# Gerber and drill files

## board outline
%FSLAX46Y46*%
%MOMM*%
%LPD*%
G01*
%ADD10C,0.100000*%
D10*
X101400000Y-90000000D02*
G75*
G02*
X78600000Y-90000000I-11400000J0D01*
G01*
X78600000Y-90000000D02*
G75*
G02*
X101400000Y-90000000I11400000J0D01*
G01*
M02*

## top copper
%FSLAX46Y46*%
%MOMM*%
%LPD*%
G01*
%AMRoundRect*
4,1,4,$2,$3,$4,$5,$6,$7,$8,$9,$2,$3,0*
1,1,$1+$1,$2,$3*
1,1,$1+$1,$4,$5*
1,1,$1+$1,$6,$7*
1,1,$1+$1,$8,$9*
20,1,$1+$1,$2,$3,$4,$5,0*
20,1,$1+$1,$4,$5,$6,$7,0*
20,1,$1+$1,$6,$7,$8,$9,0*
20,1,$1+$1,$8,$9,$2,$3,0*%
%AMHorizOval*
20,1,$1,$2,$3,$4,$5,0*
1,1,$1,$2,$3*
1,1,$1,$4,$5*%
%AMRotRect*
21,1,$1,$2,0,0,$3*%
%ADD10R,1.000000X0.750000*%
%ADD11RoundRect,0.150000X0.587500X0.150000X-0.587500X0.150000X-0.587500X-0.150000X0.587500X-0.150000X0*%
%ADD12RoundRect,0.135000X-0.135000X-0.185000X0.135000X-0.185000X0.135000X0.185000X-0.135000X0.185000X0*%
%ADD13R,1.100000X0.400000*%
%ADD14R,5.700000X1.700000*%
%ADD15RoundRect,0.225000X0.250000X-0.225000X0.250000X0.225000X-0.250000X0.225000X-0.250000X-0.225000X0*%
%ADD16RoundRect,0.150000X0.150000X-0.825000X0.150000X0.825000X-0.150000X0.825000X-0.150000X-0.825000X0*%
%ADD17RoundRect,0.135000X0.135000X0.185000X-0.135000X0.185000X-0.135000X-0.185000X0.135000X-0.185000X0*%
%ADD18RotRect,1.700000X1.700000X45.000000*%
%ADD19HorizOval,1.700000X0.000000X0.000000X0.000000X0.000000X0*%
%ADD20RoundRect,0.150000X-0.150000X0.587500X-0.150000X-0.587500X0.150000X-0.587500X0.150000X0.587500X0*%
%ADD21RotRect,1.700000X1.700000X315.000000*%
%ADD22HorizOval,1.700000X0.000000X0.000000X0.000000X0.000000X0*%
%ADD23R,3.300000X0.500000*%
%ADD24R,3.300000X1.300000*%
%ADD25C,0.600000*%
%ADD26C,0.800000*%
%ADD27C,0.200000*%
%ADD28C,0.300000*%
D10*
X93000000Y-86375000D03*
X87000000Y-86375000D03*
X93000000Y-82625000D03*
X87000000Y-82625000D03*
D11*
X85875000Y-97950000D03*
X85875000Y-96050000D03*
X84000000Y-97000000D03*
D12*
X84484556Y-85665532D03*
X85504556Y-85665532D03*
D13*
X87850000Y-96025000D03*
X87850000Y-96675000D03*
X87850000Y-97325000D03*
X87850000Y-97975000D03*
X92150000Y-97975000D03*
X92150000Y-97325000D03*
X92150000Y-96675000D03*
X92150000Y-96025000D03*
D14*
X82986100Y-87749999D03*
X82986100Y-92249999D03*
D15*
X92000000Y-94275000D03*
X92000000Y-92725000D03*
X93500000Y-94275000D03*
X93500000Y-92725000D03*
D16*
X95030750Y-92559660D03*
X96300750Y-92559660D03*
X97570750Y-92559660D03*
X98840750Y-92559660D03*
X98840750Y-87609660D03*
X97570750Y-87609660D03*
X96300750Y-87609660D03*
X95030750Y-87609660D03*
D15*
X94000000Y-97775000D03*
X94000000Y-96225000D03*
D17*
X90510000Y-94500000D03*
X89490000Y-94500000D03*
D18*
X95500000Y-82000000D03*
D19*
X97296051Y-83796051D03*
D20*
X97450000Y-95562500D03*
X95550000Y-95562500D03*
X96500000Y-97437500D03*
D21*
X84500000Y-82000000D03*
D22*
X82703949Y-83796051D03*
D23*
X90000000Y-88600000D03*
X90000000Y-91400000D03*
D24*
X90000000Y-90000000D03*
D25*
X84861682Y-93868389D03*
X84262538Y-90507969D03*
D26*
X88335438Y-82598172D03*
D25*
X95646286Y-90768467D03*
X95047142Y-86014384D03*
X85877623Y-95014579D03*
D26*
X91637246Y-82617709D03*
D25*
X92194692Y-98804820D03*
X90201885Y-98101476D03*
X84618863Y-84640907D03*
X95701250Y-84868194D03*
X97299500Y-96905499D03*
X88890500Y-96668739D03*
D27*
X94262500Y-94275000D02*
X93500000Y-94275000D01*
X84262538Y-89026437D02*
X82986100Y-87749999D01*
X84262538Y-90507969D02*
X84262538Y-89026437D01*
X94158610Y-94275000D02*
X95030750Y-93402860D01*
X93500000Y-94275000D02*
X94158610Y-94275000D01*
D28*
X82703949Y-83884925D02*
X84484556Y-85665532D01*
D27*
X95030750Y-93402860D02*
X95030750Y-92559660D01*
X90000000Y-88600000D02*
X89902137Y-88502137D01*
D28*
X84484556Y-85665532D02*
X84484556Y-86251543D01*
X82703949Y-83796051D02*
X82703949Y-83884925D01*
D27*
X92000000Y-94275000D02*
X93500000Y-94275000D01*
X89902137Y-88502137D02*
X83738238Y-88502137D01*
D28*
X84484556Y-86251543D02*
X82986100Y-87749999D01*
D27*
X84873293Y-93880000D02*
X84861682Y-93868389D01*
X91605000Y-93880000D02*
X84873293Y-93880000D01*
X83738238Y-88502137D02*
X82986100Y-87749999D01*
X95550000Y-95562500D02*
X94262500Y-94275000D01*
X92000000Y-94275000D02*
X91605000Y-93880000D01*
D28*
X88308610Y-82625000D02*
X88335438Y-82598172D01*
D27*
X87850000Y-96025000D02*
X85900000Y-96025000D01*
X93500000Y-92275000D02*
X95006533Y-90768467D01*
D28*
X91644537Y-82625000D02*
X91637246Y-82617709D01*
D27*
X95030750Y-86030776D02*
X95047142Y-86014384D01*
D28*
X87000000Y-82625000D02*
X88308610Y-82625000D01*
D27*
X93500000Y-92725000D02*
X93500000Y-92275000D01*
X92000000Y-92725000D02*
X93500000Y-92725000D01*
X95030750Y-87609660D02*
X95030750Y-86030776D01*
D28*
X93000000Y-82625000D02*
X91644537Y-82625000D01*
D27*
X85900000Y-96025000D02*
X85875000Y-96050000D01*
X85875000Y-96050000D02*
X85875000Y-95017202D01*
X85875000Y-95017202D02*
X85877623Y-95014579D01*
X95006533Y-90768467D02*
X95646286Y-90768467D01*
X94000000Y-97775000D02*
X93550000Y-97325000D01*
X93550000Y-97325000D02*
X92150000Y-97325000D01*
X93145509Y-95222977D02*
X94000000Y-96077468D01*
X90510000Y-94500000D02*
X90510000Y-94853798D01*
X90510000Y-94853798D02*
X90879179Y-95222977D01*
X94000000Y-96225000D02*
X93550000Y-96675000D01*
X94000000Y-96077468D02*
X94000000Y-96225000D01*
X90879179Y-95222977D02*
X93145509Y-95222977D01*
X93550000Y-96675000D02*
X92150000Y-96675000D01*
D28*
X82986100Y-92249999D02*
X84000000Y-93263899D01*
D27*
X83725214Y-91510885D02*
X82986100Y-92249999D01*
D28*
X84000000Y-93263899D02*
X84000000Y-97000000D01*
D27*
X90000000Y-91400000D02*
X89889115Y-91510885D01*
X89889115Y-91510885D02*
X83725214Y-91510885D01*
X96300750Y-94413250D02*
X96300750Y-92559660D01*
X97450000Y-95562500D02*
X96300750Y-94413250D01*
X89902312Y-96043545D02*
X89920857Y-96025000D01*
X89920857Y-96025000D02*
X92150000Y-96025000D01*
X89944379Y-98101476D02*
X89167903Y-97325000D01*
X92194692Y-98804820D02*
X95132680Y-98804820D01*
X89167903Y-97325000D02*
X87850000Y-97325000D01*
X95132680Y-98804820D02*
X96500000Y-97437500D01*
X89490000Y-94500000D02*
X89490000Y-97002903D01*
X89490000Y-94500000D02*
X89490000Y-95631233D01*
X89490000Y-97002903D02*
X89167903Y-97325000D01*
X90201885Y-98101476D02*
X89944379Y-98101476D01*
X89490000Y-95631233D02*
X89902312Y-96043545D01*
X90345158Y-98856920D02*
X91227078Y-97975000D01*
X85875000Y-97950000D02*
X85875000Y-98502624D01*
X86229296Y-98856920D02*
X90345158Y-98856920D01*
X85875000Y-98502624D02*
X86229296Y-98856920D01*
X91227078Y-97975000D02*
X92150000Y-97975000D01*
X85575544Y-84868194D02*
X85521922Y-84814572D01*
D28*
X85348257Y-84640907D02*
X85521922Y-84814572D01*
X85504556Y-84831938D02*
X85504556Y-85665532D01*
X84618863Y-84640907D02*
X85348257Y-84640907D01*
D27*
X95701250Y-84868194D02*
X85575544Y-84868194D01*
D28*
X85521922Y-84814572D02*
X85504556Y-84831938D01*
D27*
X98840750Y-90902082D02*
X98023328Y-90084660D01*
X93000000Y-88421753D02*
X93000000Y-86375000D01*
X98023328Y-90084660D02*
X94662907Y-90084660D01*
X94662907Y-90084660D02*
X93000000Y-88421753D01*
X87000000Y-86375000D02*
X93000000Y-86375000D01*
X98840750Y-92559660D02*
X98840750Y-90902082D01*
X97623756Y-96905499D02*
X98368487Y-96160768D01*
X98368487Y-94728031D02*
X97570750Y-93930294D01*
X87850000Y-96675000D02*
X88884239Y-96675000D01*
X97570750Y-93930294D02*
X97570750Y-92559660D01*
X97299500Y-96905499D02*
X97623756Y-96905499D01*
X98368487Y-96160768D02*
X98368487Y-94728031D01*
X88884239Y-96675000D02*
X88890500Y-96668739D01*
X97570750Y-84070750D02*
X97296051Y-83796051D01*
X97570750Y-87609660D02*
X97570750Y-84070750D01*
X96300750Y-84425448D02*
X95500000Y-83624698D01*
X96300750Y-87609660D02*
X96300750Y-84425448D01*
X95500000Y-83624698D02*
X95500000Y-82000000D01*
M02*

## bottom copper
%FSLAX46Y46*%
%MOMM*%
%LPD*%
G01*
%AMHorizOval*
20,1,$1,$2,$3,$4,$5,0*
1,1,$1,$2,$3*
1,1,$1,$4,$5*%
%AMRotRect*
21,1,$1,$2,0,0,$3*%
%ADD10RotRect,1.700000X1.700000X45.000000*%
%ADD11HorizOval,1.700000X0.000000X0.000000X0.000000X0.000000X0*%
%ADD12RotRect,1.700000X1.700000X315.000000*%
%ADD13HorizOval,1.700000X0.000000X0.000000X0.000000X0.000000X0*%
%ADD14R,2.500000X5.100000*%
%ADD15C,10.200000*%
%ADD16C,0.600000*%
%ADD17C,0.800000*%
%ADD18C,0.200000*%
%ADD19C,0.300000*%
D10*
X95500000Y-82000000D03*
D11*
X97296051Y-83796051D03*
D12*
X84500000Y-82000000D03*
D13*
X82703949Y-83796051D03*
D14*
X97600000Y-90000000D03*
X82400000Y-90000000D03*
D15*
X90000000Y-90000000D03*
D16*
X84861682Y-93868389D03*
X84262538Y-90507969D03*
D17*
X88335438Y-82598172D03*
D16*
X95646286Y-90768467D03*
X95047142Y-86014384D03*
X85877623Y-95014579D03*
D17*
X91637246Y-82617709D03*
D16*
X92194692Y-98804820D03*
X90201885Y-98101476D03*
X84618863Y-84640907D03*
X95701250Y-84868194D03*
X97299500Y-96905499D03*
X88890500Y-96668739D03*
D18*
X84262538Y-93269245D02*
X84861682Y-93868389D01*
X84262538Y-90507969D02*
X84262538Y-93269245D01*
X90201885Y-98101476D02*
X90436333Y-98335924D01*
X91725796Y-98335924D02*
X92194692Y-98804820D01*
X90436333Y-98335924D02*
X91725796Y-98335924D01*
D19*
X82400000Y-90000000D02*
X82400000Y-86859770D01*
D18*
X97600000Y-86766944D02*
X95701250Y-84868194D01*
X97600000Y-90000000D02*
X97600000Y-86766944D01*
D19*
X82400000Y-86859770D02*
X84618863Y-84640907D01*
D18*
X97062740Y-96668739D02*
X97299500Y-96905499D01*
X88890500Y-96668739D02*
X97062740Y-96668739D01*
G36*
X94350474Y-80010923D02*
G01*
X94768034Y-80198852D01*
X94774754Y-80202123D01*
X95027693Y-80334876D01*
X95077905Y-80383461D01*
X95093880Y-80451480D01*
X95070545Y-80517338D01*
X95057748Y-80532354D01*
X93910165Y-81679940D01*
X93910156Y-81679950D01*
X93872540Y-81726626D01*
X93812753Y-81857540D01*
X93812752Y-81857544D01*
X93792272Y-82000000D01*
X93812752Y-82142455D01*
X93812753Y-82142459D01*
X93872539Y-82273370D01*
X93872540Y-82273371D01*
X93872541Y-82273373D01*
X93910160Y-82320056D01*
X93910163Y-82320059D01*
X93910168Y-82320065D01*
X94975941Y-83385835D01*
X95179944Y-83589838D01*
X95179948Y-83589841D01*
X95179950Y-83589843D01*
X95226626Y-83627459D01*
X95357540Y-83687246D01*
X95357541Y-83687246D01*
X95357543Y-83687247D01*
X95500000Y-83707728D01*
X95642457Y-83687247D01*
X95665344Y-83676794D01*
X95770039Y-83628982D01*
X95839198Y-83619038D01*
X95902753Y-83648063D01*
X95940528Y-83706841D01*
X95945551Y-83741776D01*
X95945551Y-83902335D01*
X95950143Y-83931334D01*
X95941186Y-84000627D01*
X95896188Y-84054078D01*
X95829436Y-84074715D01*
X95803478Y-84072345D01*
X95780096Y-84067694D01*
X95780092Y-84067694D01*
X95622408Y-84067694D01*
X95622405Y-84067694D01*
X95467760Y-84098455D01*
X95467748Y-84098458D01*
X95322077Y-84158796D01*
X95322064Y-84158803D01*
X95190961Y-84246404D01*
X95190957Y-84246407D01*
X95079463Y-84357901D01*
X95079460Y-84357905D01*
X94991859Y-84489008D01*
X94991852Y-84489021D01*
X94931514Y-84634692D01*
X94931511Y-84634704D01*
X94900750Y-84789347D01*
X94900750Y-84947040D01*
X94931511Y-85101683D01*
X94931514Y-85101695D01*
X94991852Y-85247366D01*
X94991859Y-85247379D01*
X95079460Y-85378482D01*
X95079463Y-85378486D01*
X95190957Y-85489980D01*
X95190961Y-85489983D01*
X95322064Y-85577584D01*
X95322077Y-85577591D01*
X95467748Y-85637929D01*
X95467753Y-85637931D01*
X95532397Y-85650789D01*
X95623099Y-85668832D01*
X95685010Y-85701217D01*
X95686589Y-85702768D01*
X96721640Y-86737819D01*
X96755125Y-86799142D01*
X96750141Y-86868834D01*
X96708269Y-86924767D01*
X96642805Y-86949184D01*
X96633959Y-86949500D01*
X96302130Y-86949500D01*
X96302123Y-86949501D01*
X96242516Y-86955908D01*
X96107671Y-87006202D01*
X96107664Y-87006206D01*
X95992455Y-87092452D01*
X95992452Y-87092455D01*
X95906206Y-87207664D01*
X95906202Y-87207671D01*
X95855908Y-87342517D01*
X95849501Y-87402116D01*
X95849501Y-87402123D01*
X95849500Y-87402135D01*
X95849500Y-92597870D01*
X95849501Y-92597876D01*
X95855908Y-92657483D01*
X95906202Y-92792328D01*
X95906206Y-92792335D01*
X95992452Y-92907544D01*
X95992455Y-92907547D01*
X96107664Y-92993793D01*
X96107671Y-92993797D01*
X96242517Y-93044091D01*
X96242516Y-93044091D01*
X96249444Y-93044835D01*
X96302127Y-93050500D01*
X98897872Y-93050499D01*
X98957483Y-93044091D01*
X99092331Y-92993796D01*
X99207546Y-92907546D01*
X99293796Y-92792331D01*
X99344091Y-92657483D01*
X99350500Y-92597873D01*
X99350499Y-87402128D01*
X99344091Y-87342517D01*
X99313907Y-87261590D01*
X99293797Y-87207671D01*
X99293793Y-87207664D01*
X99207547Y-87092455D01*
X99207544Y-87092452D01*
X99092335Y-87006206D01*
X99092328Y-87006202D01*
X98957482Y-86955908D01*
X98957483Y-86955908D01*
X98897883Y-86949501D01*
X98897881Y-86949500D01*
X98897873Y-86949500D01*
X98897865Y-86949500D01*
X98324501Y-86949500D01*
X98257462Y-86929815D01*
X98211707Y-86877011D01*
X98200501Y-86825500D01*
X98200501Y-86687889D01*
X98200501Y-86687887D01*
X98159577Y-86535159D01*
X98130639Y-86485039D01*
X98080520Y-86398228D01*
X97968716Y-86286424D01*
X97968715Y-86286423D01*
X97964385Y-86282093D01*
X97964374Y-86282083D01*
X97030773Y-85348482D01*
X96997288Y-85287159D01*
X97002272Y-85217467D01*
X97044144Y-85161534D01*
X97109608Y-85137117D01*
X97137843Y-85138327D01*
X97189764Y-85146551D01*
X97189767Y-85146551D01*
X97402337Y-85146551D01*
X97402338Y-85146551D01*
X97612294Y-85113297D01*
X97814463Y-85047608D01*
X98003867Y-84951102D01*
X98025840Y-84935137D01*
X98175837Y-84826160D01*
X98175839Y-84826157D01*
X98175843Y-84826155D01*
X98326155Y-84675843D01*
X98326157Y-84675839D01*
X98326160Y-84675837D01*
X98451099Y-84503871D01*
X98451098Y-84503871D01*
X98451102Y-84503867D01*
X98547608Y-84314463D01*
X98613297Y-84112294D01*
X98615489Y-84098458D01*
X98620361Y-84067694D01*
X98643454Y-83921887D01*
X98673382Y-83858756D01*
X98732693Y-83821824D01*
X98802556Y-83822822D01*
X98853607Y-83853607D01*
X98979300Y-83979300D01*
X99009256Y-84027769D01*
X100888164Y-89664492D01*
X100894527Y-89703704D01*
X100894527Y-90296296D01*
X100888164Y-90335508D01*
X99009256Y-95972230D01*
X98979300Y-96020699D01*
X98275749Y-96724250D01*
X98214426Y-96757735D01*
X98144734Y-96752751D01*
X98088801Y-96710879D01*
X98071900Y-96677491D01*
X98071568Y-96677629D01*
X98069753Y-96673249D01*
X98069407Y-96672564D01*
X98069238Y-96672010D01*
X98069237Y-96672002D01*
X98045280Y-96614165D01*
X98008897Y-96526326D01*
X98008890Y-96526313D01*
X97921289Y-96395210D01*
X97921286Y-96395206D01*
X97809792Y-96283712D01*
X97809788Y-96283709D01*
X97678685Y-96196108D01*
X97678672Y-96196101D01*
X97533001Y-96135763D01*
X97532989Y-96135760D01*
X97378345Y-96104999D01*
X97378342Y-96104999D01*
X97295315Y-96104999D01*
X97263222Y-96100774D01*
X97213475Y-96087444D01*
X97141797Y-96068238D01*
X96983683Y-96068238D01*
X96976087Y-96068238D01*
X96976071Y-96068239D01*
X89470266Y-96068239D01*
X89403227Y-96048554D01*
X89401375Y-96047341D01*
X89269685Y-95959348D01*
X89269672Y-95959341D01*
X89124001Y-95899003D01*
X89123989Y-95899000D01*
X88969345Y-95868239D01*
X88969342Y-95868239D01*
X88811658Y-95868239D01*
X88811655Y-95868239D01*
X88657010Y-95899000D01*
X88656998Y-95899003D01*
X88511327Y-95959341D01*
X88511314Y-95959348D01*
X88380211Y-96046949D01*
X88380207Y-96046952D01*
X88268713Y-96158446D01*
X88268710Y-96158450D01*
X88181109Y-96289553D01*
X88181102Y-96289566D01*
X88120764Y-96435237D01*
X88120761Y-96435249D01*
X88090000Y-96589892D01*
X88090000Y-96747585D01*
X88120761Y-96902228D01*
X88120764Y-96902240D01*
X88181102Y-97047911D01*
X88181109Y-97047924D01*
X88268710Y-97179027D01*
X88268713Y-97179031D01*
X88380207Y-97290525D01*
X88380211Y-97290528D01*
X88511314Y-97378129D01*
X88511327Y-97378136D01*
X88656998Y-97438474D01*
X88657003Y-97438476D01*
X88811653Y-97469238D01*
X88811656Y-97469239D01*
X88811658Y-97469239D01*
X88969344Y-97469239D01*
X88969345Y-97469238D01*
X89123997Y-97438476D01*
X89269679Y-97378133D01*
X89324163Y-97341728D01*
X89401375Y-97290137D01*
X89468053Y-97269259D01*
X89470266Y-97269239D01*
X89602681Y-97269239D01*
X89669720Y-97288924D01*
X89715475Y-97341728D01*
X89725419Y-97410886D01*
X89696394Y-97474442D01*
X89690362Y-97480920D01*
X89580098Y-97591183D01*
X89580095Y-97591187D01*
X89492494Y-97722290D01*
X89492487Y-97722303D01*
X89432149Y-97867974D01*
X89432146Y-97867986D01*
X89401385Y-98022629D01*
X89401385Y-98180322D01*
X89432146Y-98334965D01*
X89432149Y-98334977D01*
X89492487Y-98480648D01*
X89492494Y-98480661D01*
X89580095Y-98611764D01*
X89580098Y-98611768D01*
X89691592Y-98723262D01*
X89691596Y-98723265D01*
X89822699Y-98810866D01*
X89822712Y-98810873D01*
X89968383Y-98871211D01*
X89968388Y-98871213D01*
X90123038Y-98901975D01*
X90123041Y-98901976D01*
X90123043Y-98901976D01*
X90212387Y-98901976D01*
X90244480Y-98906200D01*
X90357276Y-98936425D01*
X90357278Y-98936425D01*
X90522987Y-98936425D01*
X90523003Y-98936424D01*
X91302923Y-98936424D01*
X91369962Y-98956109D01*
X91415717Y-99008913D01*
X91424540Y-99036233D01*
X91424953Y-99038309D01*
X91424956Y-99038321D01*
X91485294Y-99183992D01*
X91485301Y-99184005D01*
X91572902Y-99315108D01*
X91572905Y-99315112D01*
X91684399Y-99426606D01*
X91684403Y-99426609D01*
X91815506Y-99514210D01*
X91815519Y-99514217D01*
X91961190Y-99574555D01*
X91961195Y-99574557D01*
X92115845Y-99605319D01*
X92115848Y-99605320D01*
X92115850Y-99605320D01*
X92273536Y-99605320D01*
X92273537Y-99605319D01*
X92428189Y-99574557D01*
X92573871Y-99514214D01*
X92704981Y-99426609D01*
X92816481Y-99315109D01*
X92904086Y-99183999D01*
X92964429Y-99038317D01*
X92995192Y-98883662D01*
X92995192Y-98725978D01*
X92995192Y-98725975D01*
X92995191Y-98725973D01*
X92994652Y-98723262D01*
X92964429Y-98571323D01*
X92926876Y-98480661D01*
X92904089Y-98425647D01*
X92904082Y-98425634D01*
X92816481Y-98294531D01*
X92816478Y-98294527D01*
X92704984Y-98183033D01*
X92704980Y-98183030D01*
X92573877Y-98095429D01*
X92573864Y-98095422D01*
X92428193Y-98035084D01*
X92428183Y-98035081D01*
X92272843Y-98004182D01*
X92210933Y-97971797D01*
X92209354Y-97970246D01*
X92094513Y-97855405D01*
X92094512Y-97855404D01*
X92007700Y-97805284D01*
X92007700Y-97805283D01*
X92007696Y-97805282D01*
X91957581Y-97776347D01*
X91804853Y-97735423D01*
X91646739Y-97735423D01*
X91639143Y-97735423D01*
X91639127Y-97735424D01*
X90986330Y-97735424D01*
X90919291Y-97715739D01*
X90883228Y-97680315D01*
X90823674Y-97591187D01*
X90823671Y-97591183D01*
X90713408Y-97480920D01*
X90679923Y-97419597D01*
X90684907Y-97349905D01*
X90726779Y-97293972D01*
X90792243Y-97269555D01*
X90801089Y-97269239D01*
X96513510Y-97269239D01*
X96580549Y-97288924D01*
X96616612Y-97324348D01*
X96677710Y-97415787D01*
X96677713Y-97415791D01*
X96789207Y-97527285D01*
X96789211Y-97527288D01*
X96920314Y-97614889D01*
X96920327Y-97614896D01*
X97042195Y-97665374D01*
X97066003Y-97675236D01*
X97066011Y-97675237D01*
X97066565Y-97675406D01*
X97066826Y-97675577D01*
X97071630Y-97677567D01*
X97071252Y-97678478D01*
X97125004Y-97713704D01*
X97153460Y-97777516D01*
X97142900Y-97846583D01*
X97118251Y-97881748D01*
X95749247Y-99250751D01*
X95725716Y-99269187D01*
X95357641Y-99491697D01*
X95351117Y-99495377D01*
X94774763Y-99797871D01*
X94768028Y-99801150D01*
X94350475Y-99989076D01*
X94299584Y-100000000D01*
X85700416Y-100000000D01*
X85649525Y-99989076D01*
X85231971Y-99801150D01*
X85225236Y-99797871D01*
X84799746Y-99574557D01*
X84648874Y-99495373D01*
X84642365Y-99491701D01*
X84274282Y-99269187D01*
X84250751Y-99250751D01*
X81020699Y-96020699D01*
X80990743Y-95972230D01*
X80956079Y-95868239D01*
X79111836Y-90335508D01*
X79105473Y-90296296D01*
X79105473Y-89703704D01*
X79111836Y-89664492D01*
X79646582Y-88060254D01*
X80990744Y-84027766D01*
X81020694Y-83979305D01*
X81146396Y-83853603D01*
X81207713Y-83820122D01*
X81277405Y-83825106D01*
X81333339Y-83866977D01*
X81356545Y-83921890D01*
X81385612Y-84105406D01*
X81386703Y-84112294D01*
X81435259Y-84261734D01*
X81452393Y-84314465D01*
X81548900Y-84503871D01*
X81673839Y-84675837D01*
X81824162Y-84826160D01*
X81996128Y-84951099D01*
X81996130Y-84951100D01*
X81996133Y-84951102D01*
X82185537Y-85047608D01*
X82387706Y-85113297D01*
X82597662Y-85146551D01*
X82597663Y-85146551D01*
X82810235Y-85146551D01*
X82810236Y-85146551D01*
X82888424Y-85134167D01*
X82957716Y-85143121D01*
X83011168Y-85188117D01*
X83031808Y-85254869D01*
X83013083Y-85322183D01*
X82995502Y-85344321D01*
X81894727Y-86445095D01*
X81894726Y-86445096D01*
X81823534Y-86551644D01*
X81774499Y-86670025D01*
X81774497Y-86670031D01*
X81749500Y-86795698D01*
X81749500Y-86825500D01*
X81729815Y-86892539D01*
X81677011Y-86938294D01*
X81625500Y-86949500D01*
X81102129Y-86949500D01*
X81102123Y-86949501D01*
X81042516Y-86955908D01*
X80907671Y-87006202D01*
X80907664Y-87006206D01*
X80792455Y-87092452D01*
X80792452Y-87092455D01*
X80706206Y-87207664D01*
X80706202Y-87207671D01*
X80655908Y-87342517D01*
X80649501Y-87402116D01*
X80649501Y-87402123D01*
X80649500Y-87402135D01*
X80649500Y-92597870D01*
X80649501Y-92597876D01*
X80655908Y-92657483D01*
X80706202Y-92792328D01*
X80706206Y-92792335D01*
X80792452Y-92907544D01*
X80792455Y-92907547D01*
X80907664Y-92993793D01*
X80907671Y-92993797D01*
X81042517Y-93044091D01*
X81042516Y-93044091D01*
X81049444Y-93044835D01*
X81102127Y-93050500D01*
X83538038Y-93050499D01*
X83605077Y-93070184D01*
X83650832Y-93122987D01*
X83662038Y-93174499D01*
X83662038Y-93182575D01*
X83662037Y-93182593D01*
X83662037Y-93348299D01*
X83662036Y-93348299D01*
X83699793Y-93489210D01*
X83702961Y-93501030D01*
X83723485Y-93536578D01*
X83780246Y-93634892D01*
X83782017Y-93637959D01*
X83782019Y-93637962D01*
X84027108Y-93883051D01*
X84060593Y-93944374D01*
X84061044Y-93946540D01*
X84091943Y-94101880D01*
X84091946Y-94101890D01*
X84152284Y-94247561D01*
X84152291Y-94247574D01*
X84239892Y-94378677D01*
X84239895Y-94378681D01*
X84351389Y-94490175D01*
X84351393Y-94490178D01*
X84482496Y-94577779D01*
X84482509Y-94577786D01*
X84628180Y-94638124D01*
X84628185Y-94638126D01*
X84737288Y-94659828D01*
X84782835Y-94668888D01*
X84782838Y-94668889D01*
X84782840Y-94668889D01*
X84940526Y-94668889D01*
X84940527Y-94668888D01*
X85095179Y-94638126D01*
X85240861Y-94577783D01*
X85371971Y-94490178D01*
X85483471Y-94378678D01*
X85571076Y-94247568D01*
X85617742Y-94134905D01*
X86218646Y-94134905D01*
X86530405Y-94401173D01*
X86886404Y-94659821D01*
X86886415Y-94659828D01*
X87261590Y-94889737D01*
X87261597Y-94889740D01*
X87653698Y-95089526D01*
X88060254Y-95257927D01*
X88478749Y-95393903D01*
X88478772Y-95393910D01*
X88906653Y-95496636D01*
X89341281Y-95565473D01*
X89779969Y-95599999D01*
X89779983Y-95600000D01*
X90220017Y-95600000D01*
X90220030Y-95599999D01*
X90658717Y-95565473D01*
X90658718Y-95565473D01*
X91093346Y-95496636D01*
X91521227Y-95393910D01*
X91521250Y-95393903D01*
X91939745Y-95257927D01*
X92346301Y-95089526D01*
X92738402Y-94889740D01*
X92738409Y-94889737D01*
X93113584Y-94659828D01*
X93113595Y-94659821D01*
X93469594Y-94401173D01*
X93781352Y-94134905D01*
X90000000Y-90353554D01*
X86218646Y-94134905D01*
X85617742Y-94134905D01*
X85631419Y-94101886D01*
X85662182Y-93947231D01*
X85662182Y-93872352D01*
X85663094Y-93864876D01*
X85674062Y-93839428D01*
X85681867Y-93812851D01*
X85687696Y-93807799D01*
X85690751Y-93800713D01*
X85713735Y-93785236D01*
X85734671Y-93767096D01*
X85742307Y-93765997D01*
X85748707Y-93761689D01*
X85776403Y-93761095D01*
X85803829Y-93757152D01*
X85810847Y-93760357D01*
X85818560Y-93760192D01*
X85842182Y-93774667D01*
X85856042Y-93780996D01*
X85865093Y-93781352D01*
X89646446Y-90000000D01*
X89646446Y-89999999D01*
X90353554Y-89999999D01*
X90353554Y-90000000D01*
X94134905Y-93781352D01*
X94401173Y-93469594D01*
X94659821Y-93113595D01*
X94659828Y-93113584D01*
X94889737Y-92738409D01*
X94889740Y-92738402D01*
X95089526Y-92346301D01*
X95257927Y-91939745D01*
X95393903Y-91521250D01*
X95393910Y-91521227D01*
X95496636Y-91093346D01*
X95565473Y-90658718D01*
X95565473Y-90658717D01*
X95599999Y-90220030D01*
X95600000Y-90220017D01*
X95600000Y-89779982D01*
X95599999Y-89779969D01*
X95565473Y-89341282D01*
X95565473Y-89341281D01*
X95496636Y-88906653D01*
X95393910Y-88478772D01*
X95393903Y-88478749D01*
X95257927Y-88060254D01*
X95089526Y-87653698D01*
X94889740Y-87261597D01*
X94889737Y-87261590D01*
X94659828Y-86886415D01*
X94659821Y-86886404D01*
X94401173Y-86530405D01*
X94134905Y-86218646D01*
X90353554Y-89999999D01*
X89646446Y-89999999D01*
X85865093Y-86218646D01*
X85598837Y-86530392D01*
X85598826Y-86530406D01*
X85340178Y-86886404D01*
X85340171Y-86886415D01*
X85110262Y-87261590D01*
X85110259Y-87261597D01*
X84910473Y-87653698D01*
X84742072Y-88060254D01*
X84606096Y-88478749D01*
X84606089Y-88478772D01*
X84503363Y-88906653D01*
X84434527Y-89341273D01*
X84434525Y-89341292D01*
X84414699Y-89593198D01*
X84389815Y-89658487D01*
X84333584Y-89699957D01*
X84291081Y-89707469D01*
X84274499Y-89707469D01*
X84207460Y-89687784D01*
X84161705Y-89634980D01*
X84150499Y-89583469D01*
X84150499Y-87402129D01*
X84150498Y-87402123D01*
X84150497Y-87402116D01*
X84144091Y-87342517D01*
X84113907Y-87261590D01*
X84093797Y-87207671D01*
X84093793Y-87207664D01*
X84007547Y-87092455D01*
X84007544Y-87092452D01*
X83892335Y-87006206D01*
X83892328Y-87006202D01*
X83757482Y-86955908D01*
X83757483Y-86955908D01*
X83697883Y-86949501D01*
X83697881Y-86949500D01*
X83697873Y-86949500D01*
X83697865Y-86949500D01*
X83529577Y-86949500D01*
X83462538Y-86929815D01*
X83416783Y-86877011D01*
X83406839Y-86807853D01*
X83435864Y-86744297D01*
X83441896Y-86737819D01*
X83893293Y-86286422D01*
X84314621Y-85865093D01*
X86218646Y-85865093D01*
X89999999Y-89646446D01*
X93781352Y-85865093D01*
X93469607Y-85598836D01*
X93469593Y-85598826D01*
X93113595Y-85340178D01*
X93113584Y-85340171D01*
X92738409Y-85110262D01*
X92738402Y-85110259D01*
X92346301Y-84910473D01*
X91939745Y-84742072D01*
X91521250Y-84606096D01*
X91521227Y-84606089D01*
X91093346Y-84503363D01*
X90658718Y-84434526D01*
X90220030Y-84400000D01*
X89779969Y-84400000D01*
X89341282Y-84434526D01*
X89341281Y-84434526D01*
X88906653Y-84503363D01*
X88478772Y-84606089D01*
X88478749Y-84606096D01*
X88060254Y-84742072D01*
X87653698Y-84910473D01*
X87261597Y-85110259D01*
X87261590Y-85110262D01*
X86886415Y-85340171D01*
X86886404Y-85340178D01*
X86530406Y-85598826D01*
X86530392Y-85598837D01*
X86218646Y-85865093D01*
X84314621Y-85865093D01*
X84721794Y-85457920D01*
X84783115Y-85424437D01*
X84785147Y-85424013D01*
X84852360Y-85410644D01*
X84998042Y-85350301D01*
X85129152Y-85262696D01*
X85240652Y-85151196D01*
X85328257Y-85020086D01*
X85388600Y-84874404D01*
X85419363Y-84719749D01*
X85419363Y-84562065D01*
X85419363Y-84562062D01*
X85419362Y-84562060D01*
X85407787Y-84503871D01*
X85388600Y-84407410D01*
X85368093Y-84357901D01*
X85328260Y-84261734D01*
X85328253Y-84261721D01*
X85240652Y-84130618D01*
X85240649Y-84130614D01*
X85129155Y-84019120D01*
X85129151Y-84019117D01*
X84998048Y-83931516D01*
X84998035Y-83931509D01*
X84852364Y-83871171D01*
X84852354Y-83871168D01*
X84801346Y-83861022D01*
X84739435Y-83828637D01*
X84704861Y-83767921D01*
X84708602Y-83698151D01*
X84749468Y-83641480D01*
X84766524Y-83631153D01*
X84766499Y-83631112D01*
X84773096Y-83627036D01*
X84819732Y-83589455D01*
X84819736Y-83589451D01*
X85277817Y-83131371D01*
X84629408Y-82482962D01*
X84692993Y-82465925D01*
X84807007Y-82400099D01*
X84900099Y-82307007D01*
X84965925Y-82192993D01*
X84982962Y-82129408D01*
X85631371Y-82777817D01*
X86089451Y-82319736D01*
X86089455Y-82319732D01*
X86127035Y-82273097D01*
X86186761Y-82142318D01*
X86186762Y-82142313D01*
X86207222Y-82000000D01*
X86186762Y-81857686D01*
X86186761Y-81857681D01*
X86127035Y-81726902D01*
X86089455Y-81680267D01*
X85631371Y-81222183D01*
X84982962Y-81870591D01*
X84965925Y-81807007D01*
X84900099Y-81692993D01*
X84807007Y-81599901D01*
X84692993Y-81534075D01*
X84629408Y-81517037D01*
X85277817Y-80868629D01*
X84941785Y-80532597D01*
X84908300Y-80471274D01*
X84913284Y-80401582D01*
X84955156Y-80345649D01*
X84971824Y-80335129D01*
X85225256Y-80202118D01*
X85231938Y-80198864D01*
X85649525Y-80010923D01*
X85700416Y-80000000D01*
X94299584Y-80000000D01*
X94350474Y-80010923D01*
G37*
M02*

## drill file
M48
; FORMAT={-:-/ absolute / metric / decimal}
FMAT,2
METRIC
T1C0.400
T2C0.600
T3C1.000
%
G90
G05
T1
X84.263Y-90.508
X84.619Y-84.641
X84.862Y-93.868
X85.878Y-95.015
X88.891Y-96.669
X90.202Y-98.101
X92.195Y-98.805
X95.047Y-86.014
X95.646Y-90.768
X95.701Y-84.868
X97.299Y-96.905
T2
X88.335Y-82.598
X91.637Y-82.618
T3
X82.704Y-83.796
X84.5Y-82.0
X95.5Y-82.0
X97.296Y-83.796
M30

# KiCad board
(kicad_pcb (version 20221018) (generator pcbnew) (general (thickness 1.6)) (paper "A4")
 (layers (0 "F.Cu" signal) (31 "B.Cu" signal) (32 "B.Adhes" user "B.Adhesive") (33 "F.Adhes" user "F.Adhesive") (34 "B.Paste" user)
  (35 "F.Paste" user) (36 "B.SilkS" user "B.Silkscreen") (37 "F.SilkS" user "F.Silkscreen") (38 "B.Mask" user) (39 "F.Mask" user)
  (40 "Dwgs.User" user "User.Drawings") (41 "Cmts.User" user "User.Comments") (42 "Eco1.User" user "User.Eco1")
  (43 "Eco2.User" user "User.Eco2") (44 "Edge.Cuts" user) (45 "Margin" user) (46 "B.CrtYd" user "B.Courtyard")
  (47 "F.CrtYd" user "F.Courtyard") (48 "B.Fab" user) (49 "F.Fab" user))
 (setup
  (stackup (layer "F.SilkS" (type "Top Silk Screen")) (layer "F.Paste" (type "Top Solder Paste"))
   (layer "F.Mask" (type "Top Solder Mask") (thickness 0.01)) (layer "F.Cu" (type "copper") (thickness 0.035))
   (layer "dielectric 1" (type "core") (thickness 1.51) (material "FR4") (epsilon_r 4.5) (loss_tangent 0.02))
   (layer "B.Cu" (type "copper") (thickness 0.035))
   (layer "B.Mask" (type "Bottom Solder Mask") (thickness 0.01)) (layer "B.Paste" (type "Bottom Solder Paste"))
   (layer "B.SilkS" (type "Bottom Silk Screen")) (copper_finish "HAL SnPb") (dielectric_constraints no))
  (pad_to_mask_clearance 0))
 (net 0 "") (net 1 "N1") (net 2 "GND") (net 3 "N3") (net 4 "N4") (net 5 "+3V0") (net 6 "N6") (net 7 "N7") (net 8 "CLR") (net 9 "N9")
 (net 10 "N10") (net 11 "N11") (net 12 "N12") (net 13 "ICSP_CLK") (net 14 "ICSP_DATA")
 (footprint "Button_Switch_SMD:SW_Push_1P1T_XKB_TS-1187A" (layer "F.Cu") (at 90 84.5 180)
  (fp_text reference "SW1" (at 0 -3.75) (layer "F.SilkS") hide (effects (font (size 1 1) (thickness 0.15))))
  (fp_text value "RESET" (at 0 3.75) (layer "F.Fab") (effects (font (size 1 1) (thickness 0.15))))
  (pad "1" smd rect (at -3 -1.875 180) (size 1 0.75) (layers "F.Cu" "F.Paste" "F.Mask") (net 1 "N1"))
  (pad "1" smd rect (at 3 -1.875 180) (size 1 0.75) (layers "F.Cu" "F.Paste" "F.Mask") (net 1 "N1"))
  (pad "2" smd rect (at -3 1.875 180) (size 1 0.75) (layers "F.Cu" "F.Paste" "F.Mask") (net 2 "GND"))
  (pad "2" smd rect (at 3 1.875 180) (size 1 0.75) (layers "F.Cu" "F.Paste" "F.Mask") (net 2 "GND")))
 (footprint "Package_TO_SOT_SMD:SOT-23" (layer "F.Cu") (at 84.9375 97 180)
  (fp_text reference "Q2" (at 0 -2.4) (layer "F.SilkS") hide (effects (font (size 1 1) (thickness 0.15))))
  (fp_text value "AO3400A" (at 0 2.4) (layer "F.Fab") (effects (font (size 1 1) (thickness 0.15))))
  (pad "1" smd roundrect (at -0.9375 -0.95 180) (size 1.475 0.6) (layers "F.Cu" "F.Paste" "F.Mask") (roundrect_rratio 0.25) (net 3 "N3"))
  (pad "2" smd roundrect (at -0.9375 0.95 180) (size 1.475 0.6) (layers "F.Cu" "F.Paste" "F.Mask") (roundrect_rratio 0.25) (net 2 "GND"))
  (pad "3" smd roundrect (at 0.9375 0 180) (size 1.475 0.6) (layers "F.Cu" "F.Paste" "F.Mask") (roundrect_rratio 0.25) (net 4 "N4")))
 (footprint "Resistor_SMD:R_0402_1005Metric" (layer "F.Cu") (at 84.994556 85.665532)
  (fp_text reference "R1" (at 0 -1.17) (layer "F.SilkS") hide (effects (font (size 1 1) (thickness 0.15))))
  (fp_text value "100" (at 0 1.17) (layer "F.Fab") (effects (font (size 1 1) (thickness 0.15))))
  (pad "1" smd roundrect (at -0.51 0) (size 0.54 0.64) (layers "F.Cu" "F.Paste" "F.Mask") (roundrect_rratio 0.25) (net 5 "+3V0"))
  (pad "2" smd roundrect (at 0.51 0) (size 0.54 0.64) (layers "F.Cu" "F.Paste" "F.Mask") (roundrect_rratio 0.25) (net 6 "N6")))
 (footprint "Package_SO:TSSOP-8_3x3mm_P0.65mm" (layer "F.Cu") (at 90 97)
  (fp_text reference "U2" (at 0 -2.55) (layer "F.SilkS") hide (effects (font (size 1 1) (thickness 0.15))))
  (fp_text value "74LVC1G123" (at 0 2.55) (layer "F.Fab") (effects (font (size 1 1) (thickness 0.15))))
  (pad "1" smd rect (at -2.15 -0.975) (size 1.1 0.4) (layers "F.Cu" "F.Paste" "F.Mask") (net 2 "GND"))
  (pad "2" smd rect (at -2.15 -0.325) (size 1.1 0.4) (layers "F.Cu" "F.Paste" "F.Mask") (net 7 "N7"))
  (pad "3" smd rect (at -2.15 0.325) (size 1.1 0.4) (layers "F.Cu" "F.Paste" "F.Mask") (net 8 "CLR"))
  (pad "4" smd rect (at -2.15 0.975) (size 1.1 0.4) (layers "F.Cu" "F.Paste" "F.Mask") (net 2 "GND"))
  (pad "5" smd rect (at 2.15 0.975) (size 1.1 0.4) (layers "F.Cu" "F.Paste" "F.Mask") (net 3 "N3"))
  (pad "6" smd rect (at 2.15 0.325) (size 1.1 0.4) (layers "F.Cu" "F.Paste" "F.Mask") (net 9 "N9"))
  (pad "7" smd rect (at 2.15 -0.325) (size 1.1 0.4) (layers "F.Cu" "F.Paste" "F.Mask") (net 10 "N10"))
  (pad "8" smd rect (at 2.15 -0.975) (size 1.1 0.4) (layers "F.Cu" "F.Paste" "F.Mask") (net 8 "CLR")))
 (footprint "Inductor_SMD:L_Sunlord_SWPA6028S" (layer "F.Cu") (at 82.9861 89.999999 -90)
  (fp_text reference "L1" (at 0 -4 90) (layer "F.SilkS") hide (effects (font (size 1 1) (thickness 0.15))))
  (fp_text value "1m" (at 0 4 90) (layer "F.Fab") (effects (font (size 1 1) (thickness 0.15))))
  (pad "1" smd rect (at -2.25 0 270) (size 1.7 5.7) (layers "F.Cu" "F.Paste" "F.Mask") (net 5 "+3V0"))
  (pad "2" smd rect (at 2.25 0 270) (size 1.7 5.7) (layers "F.Cu" "F.Paste" "F.Mask") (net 4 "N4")))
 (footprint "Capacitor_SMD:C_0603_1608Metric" (layer "F.Cu") (at 92 93.5 90)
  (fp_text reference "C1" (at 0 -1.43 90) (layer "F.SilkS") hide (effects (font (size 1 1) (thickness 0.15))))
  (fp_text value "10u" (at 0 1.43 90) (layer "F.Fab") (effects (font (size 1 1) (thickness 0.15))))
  (pad "1" smd roundrect (at -0.775 0 90) (size 0.9 0.95) (layers "F.Cu" "F.Paste" "F.Mask") (roundrect_rratio 0.25) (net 5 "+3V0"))
  (pad "2" smd roundrect (at 0.775 0 90) (size 0.9 0.95) (layers "F.Cu" "F.Paste" "F.Mask") (roundrect_rratio 0.25) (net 2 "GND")))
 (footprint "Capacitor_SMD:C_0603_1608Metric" (layer "F.Cu") (at 93.5 93.5 90)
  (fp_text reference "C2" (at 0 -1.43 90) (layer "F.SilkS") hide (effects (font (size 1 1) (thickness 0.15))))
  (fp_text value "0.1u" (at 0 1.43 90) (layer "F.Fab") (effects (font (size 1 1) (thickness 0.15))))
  (pad "1" smd roundrect (at -0.775 0 90) (size 0.9 0.95) (layers "F.Cu" "F.Paste" "F.Mask") (roundrect_rratio 0.25) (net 5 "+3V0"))
  (pad "2" smd roundrect (at 0.775 0 90) (size 0.9 0.95) (layers "F.Cu" "F.Paste" "F.Mask") (roundrect_rratio 0.25) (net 2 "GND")))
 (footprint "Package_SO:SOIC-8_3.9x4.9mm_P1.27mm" (layer "F.Cu") (at 96.93575 90.08466 90)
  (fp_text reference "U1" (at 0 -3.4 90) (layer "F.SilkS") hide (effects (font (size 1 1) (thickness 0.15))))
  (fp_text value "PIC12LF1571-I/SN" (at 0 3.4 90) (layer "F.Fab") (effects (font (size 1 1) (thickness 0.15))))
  (pad "1" smd roundrect (at -2.475 -1.905 90) (size 1.95 0.6) (layers "F.Cu" "F.Paste" "F.Mask") (roundrect_rratio 0.25) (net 5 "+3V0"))
  (pad "2" smd roundrect (at -2.475 -0.635 90) (size 1.95 0.6) (layers "F.Cu" "F.Paste" "F.Mask") (roundrect_rratio 0.25) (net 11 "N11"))
  (pad "3" smd roundrect (at -2.475 0.635 90) (size 1.95 0.6) (layers "F.Cu" "F.Paste" "F.Mask") (roundrect_rratio 0.25) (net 7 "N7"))
  (pad "4" smd roundrect (at -2.475 1.905 90) (size 1.95 0.6) (layers "F.Cu" "F.Paste" "F.Mask") (roundrect_rratio 0.25) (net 1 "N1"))
  (pad "5" smd roundrect (at 2.475 1.905 90) (size 1.95 0.6) (layers "F.Cu" "F.Paste" "F.Mask") (roundrect_rratio 0.25) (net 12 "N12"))
  (pad "6" smd roundrect (at 2.475 0.635 90) (size 1.95 0.6) (layers "F.Cu" "F.Paste" "F.Mask") (roundrect_rratio 0.25) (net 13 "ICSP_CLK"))
  (pad "7" smd roundrect (at 2.475 -0.635 90) (size 1.95 0.6) (layers "F.Cu" "F.Paste" "F.Mask") (roundrect_rratio 0.25)
   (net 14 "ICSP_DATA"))
  (pad "8" smd roundrect (at 2.475 -1.905 90) (size 1.95 0.6) (layers "F.Cu" "F.Paste" "F.Mask") (roundrect_rratio 0.25) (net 2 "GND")))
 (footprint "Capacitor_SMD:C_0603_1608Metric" (layer "F.Cu") (at 94 97 90)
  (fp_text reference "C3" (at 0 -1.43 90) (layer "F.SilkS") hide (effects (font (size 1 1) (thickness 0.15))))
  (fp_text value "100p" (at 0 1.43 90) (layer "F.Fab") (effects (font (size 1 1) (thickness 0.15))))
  (pad "1" smd roundrect (at -0.775 0 90) (size 0.9 0.95) (layers "F.Cu" "F.Paste" "F.Mask") (roundrect_rratio 0.25) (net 9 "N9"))
  (pad "2" smd roundrect (at 0.775 0 90) (size 0.9 0.95) (layers "F.Cu" "F.Paste" "F.Mask") (roundrect_rratio 0.25) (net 10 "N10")))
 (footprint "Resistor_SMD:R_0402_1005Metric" (layer "F.Cu") (at 90 94.5 180)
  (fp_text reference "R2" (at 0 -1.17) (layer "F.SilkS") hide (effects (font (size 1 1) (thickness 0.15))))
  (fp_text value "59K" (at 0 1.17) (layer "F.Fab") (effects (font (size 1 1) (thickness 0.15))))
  (pad "1" smd roundrect (at -0.51 0 180) (size 0.54 0.64) (layers "F.Cu" "F.Paste" "F.Mask") (roundrect_rratio 0.25) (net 10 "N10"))
  (pad "2" smd roundrect (at 0.51 0 180) (size 0.54 0.64) (layers "F.Cu" "F.Paste" "F.Mask") (roundrect_rratio 0.25) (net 8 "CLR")))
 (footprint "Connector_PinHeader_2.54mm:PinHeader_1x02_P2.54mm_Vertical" (layer "F.Cu") (at 95.5 82 45)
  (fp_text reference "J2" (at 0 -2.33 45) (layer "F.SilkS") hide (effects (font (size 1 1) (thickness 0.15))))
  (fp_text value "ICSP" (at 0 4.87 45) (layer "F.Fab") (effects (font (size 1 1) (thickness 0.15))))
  (pad "1" thru_hole rect (at 0 0 45) (size 1.7 1.7) (drill 1) (layers "*.Cu" "*.Mask") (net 14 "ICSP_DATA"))
  (pad "2" thru_hole oval (at 0 2.54 45) (size 1.7 1.7) (drill 1) (layers "*.Cu" "*.Mask") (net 13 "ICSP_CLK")))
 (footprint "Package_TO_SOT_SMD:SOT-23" (layer "F.Cu") (at 96.5 96.5 -90)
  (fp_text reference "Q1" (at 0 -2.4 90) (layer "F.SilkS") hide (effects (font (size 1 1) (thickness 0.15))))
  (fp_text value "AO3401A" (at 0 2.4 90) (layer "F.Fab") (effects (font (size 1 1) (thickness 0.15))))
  (pad "1" smd roundrect (at -0.9375 -0.95 270) (size 1.475 0.6) (layers "F.Cu" "F.Paste" "F.Mask") (roundrect_rratio 0.25) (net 11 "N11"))
  (pad "2" smd roundrect (at -0.9375 0.95 270) (size 1.475 0.6) (layers "F.Cu" "F.Paste" "F.Mask") (roundrect_rratio 0.25) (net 5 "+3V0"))
  (pad "3" smd roundrect (at 0.9375 0 270) (size 1.475 0.6) (layers "F.Cu" "F.Paste" "F.Mask") (roundrect_rratio 0.25) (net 8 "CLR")))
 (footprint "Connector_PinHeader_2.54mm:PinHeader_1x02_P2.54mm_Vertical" (layer "F.Cu") (at 84.5 82 -45)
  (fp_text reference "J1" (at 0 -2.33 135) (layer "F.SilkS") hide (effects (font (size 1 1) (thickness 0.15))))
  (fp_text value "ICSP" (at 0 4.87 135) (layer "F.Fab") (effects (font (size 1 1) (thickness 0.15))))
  (pad "1" thru_hole rect (at 0 0 315) (size 1.7 1.7) (drill 1) (layers "*.Cu" "*.Mask") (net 2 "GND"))
  (pad "2" thru_hole oval (at 0 2.54 315) (size 1.7 1.7) (drill 1) (layers "*.Cu" "*.Mask") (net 5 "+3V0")))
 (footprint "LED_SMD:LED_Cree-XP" (layer "F.Cu") (at 90 90 -90)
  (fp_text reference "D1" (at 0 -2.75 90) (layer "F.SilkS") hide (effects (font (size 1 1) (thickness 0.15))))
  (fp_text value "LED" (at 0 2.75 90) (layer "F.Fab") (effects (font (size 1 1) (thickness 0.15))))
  (pad "" smd rect (at 0 -1 270) (size 1.01 0.75) (layers "F.Paste"))
  (pad "" smd rect (at 0 0 270) (size 1.01 0.75) (layers "F.Paste"))
  (pad "" smd rect (at 0 1 270) (size 1.01 0.75) (layers "F.Paste"))
  (pad "1" smd rect (at -1.4 0 270) (size 0.5 3.3) (layers "F.Cu" "F.Paste" "F.Mask") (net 5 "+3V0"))
  (pad "2" smd rect (at 1.4 0 270) (size 0.5 3.3) (layers "F.Cu" "F.Paste" "F.Mask") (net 4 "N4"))
  (pad "3" smd rect (at 0 0 270) (size 1.3 3.3) (layers "F.Cu" "F.Mask")))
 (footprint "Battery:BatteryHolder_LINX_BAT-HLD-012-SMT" (layer "B.Cu") (at 90 90 180)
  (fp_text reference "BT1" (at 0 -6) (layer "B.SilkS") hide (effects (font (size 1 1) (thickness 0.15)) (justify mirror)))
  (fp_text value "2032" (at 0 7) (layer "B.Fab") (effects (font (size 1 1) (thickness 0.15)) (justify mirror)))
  (pad "1" smd rect (at -7.6 0 180) (size 2.5 5.1) (layers "B.Cu" "B.Paste" "B.Mask") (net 6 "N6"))
  (pad "1" smd rect (at 7.6 0 180) (size 2.5 5.1) (layers "B.Cu" "B.Paste" "B.Mask") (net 6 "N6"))
  (pad "2" smd circle (at 0 0 180) (size 10.2 10.2) (layers "B.Cu" "B.Mask") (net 2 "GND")))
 (gr_circle (center 90 90) (end 101.4 90) (stroke (width 0.1) (type default)) (fill none) (layer "Edge.Cuts"))
 (segment (start 94.2625 94.275) (end 93.5 94.275) (width 0.2) (layer "F.Cu") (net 5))
 (segment (start 84.262538 89.026437) (end 82.9861 87.749999) (width 0.2) (layer "F.Cu") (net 5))
 (segment (start 84.262538 90.507969) (end 84.262538 89.026437) (width 0.2) (layer "F.Cu") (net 5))
 (segment (start 94.15861 94.275) (end 95.03075 93.40286) (width 0.2) (layer "F.Cu") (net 5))
 (segment (start 93.5 94.275) (end 94.15861 94.275) (width 0.2) (layer "F.Cu") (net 5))
 (segment (start 82.703949 83.884925) (end 84.484556 85.665532) (width 0.3) (layer "F.Cu") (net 5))
 (segment (start 95.03075 93.40286) (end 95.03075 92.55966) (width 0.2) (layer "F.Cu") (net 5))
 (segment (start 90 88.6) (end 89.902137 88.502137) (width 0.2) (layer "F.Cu") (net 5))
 (segment (start 84.484556 85.665532) (end 84.484556 86.251543) (width 0.3) (layer "F.Cu") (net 5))
 (segment (start 82.703949 83.796051) (end 82.703949 83.884925) (width 0.3) (layer "F.Cu") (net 5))
 (segment (start 92 94.275) (end 93.5 94.275) (width 0.2) (layer "F.Cu") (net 5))
 (segment (start 89.902137 88.502137) (end 83.738238 88.502137) (width 0.2) (layer "F.Cu") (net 5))
 (segment (start 84.484556 86.251543) (end 82.9861 87.749999) (width 0.3) (layer "F.Cu") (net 5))
 (segment (start 84.873293 93.88) (end 84.861682 93.868389) (width 0.2) (layer "F.Cu") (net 5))
 (segment (start 91.605 93.88) (end 84.873293 93.88) (width 0.2) (layer "F.Cu") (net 5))
 (segment (start 83.738238 88.502137) (end 82.9861 87.749999) (width 0.2) (layer "F.Cu") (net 5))
 (segment (start 95.55 95.5625) (end 94.2625 94.275) (width 0.2) (layer "F.Cu") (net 5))
 (segment (start 92 94.275) (end 91.605 93.88) (width 0.2) (layer "F.Cu") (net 5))
 (via (at 84.861682 93.868389) (size 0.6) (drill 0.4) (layers "F.Cu" "B.Cu") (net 5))
 (via (at 84.262538 90.507969) (size 0.6) (drill 0.4) (layers "F.Cu" "B.Cu") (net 5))
 (segment (start 84.262538 93.269245) (end 84.861682 93.868389) (width 0.2) (layer "B.Cu") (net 5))
 (segment (start 84.262538 90.507969) (end 84.262538 93.269245) (width 0.2) (layer "B.Cu") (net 5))
 (segment (start 88.30861 82.625) (end 88.335438 82.598172) (width 0.3) (layer "F.Cu") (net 2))
 (segment (start 87.85 96.025) (end 85.9 96.025) (width 0.2) (layer "F.Cu") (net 2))
 (segment (start 93.5 92.275) (end 95.006533 90.768467) (width 0.2) (layer "F.Cu") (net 2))
 (segment (start 91.644537 82.625) (end 91.637246 82.617709) (width 0.3) (layer "F.Cu") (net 2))
 (segment (start 95.03075 86.030776) (end 95.047142 86.014384) (width 0.2) (layer "F.Cu") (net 2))
 (segment (start 87 82.625) (end 88.30861 82.625) (width 0.3) (layer "F.Cu") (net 2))
 (segment (start 93.5 92.725) (end 93.5 92.275) (width 0.2) (layer "F.Cu") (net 2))
 (segment (start 92 92.725) (end 93.5 92.725) (width 0.2) (layer "F.Cu") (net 2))
 (segment (start 95.03075 87.60966) (end 95.03075 86.030776) (width 0.2) (layer "F.Cu") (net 2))
 (segment (start 93 82.625) (end 91.644537 82.625) (width 0.3) (layer "F.Cu") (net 2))
 (segment (start 85.9 96.025) (end 85.875 96.05) (width 0.2) (layer "F.Cu") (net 2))
 (segment (start 85.875 96.05) (end 85.875 95.017202) (width 0.2) (layer "F.Cu") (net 2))
 (segment (start 85.875 95.017202) (end 85.877623 95.014579) (width 0.2) (layer "F.Cu") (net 2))
 (segment (start 95.006533 90.768467) (end 95.646286 90.768467) (width 0.2) (layer "F.Cu") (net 2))
 (via (at 88.335438 82.598172) (size 0.8) (drill 0.6) (layers "F.Cu" "B.Cu") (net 2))
 (via (at 95.646286 90.768467) (size 0.6) (drill 0.4) (layers "F.Cu" "B.Cu") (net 2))
 (via (at 95.047142 86.014384) (size 0.6) (drill 0.4) (layers "F.Cu" "B.Cu") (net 2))
 (via (at 85.877623 95.014579) (size 0.6) (drill 0.4) (layers "F.Cu" "B.Cu") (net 2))
 (via (at 91.637246 82.617709) (size 0.8) (drill 0.6) (layers "F.Cu" "B.Cu") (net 2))
 (segment (start 94 97.775) (end 93.55 97.325) (width 0.2) (layer "F.Cu") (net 9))
 (segment (start 93.55 97.325) (end 92.15 97.325) (width 0.2) (layer "F.Cu") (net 9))
 (segment (start 93.145509 95.222977) (end 94 96.077468) (width 0.2) (layer "F.Cu") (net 10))
 (segment (start 90.51 94.5) (end 90.51 94.853798) (width 0.2) (layer "F.Cu") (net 10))
 (segment (start 90.51 94.853798) (end 90.879179 95.222977) (width 0.2) (layer "F.Cu") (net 10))
 (segment (start 94 96.225) (end 93.55 96.675) (width 0.2) (layer "F.Cu") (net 10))
 (segment (start 94 96.077468) (end 94 96.225) (width 0.2) (layer "F.Cu") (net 10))
 (segment (start 90.879179 95.222977) (end 93.145509 95.222977) (width 0.2) (layer "F.Cu") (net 10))
 (segment (start 93.55 96.675) (end 92.15 96.675) (width 0.2) (layer "F.Cu") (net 10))
 (segment (start 82.9861 92.249999) (end 84 93.263899) (width 0.3) (layer "F.Cu") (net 4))
 (segment (start 83.725214 91.510885) (end 82.9861 92.249999) (width 0.2) (layer "F.Cu") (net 4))
 (segment (start 84 93.263899) (end 84 97) (width 0.3) (layer "F.Cu") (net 4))
 (segment (start 90 91.4) (end 89.889115 91.510885) (width 0.2) (layer "F.Cu") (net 4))
 (segment (start 89.889115 91.510885) (end 83.725214 91.510885) (width 0.2) (layer "F.Cu") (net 4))
 (segment (start 96.30075 94.41325) (end 96.30075 92.55966) (width 0.2) (layer "F.Cu") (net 11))
 (segment (start 97.45 95.5625) (end 96.30075 94.41325) (width 0.2) (layer "F.Cu") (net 11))
 (segment (start 89.902312 96.043545) (end 89.920857 96.025) (width 0.2) (layer "F.Cu") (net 8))
 (segment (start 89.920857 96.025) (end 92.15 96.025) (width 0.2) (layer "F.Cu") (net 8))
 (segment (start 89.944379 98.101476) (end 89.167903 97.325) (width 0.2) (layer "F.Cu") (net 8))
 (segment (start 92.194692 98.80482) (end 95.13268 98.80482) (width 0.2) (layer "F.Cu") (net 8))
 (segment (start 89.167903 97.325) (end 87.85 97.325) (width 0.2) (layer "F.Cu") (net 8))
 (segment (start 95.13268 98.80482) (end 96.5 97.4375) (width 0.2) (layer "F.Cu") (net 8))
 (segment (start 89.49 94.5) (end 89.49 97.002903) (width 0.2) (layer "F.Cu") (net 8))
 (segment (start 89.49 94.5) (end 89.49 95.631233) (width 0.2) (layer "F.Cu") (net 8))
 (segment (start 89.49 97.002903) (end 89.167903 97.325) (width 0.2) (layer "F.Cu") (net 8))
 (segment (start 90.201885 98.101476) (end 89.944379 98.101476) (width 0.2) (layer "F.Cu") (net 8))
 (segment (start 89.49 95.631233) (end 89.902312 96.043545) (width 0.2) (layer "F.Cu") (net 8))
 (via (at 92.194692 98.80482) (size 0.6) (drill 0.4) (layers "F.Cu" "B.Cu") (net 8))
 (via (at 90.201885 98.101476) (size 0.6) (drill 0.4) (layers "F.Cu" "B.Cu") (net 8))
 (segment (start 90.201885 98.101476) (end 90.436333 98.335924) (width 0.2) (layer "B.Cu") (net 8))
 (segment (start 91.725796 98.335924) (end 92.194692 98.80482) (width 0.2) (layer "B.Cu") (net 8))
 (segment (start 90.436333 98.335924) (end 91.725796 98.335924) (width 0.2) (layer "B.Cu") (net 8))
 (segment (start 90.345158 98.85692) (end 91.227078 97.975) (width 0.2) (layer "F.Cu") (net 3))
 (segment (start 85.875 97.95) (end 85.875 98.502624) (width 0.2) (layer "F.Cu") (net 3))
 (segment (start 86.229296 98.85692) (end 90.345158 98.85692) (width 0.2) (layer "F.Cu") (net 3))
 (segment (start 85.875 98.502624) (end 86.229296 98.85692) (width 0.2) (layer "F.Cu") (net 3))
 (segment (start 91.227078 97.975) (end 92.15 97.975) (width 0.2) (layer "F.Cu") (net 3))
 (segment (start 85.575544 84.868194) (end 85.521922 84.814572) (width 0.2) (layer "F.Cu") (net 6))
 (segment (start 85.348257 84.640907) (end 85.521922 84.814572) (width 0.3) (layer "F.Cu") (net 6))
 (segment (start 85.504556 84.831938) (end 85.504556 85.665532) (width 0.3) (layer "F.Cu") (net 6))
 (segment (start 84.618863 84.640907) (end 85.348257 84.640907) (width 0.3) (layer "F.Cu") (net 6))
 (segment (start 95.70125 84.868194) (end 85.575544 84.868194) (width 0.2) (layer "F.Cu") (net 6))
 (segment (start 85.521922 84.814572) (end 85.504556 84.831938) (width 0.3) (layer "F.Cu") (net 6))
 (via (at 84.618863 84.640907) (size 0.6) (drill 0.4) (layers "F.Cu" "B.Cu") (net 6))
 (via (at 95.70125 84.868194) (size 0.6) (drill 0.4) (layers "F.Cu" "B.Cu") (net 6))
 (segment (start 82.4 90) (end 82.4 86.85977) (width 0.3) (layer "B.Cu") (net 6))
 (segment (start 97.6 86.766944) (end 95.70125 84.868194) (width 0.2) (layer "B.Cu") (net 6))
 (segment (start 97.6 90) (end 97.6 86.766944) (width 0.2) (layer "B.Cu") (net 6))
 (segment (start 82.4 86.85977) (end 84.618863 84.640907) (width 0.3) (layer "B.Cu") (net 6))
 (segment (start 98.84075 90.902082) (end 98.023328 90.08466) (width 0.2) (layer "F.Cu") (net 1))
 (segment (start 93 88.421753) (end 93 86.375) (width 0.2) (layer "F.Cu") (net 1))
 (segment (start 98.023328 90.08466) (end 94.662907 90.08466) (width 0.2) (layer "F.Cu") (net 1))
 (segment (start 94.662907 90.08466) (end 93 88.421753) (width 0.2) (layer "F.Cu") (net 1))
 (segment (start 87 86.375) (end 93 86.375) (width 0.2) (layer "F.Cu") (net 1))
 (segment (start 98.84075 92.55966) (end 98.84075 90.902082) (width 0.2) (layer "F.Cu") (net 1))
 (segment (start 97.623756 96.905499) (end 98.368487 96.160768) (width 0.2) (layer "F.Cu") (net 7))
 (segment (start 98.368487 94.728031) (end 97.57075 93.930294) (width 0.2) (layer "F.Cu") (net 7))
 (segment (start 87.85 96.675) (end 88.884239 96.675) (width 0.2) (layer "F.Cu") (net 7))
 (segment (start 97.57075 93.930294) (end 97.57075 92.55966) (width 0.2) (layer "F.Cu") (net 7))
 (segment (start 97.2995 96.905499) (end 97.623756 96.905499) (width 0.2) (layer "F.Cu") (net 7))
 (segment (start 98.368487 96.160768) (end 98.368487 94.728031) (width 0.2) (layer "F.Cu") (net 7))
 (segment (start 88.884239 96.675) (end 88.8905 96.668739) (width 0.2) (layer "F.Cu") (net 7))
 (via (at 97.2995 96.905499) (size 0.6) (drill 0.4) (layers "F.Cu" "B.Cu") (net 7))
 (via (at 88.8905 96.668739) (size 0.6) (drill 0.4) (layers "F.Cu" "B.Cu") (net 7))
 (segment (start 97.06274 96.668739) (end 97.2995 96.905499) (width 0.2) (layer "B.Cu") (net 7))
 (segment (start 88.8905 96.668739) (end 97.06274 96.668739) (width 0.2) (layer "B.Cu") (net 7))
 (segment (start 97.57075 84.07075) (end 97.296051 83.796051) (width 0.2) (layer "F.Cu") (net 13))
 (segment (start 97.57075 87.60966) (end 97.57075 84.07075) (width 0.2) (layer "F.Cu") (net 13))
 (segment (start 96.30075 84.425448) (end 95.5 83.624698) (width 0.2) (layer "F.Cu") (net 14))
 (segment (start 96.30075 87.60966) (end 96.30075 84.425448) (width 0.2) (layer "F.Cu") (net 14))
 (segment (start 95.5 83.624698) (end 95.5 82) (width 0.2) (layer "F.Cu") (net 14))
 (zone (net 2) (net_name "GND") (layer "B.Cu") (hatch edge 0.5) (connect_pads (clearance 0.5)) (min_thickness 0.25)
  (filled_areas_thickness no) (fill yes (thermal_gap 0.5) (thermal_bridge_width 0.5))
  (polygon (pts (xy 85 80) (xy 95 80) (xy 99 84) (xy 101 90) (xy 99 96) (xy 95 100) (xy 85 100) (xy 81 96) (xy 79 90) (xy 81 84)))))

